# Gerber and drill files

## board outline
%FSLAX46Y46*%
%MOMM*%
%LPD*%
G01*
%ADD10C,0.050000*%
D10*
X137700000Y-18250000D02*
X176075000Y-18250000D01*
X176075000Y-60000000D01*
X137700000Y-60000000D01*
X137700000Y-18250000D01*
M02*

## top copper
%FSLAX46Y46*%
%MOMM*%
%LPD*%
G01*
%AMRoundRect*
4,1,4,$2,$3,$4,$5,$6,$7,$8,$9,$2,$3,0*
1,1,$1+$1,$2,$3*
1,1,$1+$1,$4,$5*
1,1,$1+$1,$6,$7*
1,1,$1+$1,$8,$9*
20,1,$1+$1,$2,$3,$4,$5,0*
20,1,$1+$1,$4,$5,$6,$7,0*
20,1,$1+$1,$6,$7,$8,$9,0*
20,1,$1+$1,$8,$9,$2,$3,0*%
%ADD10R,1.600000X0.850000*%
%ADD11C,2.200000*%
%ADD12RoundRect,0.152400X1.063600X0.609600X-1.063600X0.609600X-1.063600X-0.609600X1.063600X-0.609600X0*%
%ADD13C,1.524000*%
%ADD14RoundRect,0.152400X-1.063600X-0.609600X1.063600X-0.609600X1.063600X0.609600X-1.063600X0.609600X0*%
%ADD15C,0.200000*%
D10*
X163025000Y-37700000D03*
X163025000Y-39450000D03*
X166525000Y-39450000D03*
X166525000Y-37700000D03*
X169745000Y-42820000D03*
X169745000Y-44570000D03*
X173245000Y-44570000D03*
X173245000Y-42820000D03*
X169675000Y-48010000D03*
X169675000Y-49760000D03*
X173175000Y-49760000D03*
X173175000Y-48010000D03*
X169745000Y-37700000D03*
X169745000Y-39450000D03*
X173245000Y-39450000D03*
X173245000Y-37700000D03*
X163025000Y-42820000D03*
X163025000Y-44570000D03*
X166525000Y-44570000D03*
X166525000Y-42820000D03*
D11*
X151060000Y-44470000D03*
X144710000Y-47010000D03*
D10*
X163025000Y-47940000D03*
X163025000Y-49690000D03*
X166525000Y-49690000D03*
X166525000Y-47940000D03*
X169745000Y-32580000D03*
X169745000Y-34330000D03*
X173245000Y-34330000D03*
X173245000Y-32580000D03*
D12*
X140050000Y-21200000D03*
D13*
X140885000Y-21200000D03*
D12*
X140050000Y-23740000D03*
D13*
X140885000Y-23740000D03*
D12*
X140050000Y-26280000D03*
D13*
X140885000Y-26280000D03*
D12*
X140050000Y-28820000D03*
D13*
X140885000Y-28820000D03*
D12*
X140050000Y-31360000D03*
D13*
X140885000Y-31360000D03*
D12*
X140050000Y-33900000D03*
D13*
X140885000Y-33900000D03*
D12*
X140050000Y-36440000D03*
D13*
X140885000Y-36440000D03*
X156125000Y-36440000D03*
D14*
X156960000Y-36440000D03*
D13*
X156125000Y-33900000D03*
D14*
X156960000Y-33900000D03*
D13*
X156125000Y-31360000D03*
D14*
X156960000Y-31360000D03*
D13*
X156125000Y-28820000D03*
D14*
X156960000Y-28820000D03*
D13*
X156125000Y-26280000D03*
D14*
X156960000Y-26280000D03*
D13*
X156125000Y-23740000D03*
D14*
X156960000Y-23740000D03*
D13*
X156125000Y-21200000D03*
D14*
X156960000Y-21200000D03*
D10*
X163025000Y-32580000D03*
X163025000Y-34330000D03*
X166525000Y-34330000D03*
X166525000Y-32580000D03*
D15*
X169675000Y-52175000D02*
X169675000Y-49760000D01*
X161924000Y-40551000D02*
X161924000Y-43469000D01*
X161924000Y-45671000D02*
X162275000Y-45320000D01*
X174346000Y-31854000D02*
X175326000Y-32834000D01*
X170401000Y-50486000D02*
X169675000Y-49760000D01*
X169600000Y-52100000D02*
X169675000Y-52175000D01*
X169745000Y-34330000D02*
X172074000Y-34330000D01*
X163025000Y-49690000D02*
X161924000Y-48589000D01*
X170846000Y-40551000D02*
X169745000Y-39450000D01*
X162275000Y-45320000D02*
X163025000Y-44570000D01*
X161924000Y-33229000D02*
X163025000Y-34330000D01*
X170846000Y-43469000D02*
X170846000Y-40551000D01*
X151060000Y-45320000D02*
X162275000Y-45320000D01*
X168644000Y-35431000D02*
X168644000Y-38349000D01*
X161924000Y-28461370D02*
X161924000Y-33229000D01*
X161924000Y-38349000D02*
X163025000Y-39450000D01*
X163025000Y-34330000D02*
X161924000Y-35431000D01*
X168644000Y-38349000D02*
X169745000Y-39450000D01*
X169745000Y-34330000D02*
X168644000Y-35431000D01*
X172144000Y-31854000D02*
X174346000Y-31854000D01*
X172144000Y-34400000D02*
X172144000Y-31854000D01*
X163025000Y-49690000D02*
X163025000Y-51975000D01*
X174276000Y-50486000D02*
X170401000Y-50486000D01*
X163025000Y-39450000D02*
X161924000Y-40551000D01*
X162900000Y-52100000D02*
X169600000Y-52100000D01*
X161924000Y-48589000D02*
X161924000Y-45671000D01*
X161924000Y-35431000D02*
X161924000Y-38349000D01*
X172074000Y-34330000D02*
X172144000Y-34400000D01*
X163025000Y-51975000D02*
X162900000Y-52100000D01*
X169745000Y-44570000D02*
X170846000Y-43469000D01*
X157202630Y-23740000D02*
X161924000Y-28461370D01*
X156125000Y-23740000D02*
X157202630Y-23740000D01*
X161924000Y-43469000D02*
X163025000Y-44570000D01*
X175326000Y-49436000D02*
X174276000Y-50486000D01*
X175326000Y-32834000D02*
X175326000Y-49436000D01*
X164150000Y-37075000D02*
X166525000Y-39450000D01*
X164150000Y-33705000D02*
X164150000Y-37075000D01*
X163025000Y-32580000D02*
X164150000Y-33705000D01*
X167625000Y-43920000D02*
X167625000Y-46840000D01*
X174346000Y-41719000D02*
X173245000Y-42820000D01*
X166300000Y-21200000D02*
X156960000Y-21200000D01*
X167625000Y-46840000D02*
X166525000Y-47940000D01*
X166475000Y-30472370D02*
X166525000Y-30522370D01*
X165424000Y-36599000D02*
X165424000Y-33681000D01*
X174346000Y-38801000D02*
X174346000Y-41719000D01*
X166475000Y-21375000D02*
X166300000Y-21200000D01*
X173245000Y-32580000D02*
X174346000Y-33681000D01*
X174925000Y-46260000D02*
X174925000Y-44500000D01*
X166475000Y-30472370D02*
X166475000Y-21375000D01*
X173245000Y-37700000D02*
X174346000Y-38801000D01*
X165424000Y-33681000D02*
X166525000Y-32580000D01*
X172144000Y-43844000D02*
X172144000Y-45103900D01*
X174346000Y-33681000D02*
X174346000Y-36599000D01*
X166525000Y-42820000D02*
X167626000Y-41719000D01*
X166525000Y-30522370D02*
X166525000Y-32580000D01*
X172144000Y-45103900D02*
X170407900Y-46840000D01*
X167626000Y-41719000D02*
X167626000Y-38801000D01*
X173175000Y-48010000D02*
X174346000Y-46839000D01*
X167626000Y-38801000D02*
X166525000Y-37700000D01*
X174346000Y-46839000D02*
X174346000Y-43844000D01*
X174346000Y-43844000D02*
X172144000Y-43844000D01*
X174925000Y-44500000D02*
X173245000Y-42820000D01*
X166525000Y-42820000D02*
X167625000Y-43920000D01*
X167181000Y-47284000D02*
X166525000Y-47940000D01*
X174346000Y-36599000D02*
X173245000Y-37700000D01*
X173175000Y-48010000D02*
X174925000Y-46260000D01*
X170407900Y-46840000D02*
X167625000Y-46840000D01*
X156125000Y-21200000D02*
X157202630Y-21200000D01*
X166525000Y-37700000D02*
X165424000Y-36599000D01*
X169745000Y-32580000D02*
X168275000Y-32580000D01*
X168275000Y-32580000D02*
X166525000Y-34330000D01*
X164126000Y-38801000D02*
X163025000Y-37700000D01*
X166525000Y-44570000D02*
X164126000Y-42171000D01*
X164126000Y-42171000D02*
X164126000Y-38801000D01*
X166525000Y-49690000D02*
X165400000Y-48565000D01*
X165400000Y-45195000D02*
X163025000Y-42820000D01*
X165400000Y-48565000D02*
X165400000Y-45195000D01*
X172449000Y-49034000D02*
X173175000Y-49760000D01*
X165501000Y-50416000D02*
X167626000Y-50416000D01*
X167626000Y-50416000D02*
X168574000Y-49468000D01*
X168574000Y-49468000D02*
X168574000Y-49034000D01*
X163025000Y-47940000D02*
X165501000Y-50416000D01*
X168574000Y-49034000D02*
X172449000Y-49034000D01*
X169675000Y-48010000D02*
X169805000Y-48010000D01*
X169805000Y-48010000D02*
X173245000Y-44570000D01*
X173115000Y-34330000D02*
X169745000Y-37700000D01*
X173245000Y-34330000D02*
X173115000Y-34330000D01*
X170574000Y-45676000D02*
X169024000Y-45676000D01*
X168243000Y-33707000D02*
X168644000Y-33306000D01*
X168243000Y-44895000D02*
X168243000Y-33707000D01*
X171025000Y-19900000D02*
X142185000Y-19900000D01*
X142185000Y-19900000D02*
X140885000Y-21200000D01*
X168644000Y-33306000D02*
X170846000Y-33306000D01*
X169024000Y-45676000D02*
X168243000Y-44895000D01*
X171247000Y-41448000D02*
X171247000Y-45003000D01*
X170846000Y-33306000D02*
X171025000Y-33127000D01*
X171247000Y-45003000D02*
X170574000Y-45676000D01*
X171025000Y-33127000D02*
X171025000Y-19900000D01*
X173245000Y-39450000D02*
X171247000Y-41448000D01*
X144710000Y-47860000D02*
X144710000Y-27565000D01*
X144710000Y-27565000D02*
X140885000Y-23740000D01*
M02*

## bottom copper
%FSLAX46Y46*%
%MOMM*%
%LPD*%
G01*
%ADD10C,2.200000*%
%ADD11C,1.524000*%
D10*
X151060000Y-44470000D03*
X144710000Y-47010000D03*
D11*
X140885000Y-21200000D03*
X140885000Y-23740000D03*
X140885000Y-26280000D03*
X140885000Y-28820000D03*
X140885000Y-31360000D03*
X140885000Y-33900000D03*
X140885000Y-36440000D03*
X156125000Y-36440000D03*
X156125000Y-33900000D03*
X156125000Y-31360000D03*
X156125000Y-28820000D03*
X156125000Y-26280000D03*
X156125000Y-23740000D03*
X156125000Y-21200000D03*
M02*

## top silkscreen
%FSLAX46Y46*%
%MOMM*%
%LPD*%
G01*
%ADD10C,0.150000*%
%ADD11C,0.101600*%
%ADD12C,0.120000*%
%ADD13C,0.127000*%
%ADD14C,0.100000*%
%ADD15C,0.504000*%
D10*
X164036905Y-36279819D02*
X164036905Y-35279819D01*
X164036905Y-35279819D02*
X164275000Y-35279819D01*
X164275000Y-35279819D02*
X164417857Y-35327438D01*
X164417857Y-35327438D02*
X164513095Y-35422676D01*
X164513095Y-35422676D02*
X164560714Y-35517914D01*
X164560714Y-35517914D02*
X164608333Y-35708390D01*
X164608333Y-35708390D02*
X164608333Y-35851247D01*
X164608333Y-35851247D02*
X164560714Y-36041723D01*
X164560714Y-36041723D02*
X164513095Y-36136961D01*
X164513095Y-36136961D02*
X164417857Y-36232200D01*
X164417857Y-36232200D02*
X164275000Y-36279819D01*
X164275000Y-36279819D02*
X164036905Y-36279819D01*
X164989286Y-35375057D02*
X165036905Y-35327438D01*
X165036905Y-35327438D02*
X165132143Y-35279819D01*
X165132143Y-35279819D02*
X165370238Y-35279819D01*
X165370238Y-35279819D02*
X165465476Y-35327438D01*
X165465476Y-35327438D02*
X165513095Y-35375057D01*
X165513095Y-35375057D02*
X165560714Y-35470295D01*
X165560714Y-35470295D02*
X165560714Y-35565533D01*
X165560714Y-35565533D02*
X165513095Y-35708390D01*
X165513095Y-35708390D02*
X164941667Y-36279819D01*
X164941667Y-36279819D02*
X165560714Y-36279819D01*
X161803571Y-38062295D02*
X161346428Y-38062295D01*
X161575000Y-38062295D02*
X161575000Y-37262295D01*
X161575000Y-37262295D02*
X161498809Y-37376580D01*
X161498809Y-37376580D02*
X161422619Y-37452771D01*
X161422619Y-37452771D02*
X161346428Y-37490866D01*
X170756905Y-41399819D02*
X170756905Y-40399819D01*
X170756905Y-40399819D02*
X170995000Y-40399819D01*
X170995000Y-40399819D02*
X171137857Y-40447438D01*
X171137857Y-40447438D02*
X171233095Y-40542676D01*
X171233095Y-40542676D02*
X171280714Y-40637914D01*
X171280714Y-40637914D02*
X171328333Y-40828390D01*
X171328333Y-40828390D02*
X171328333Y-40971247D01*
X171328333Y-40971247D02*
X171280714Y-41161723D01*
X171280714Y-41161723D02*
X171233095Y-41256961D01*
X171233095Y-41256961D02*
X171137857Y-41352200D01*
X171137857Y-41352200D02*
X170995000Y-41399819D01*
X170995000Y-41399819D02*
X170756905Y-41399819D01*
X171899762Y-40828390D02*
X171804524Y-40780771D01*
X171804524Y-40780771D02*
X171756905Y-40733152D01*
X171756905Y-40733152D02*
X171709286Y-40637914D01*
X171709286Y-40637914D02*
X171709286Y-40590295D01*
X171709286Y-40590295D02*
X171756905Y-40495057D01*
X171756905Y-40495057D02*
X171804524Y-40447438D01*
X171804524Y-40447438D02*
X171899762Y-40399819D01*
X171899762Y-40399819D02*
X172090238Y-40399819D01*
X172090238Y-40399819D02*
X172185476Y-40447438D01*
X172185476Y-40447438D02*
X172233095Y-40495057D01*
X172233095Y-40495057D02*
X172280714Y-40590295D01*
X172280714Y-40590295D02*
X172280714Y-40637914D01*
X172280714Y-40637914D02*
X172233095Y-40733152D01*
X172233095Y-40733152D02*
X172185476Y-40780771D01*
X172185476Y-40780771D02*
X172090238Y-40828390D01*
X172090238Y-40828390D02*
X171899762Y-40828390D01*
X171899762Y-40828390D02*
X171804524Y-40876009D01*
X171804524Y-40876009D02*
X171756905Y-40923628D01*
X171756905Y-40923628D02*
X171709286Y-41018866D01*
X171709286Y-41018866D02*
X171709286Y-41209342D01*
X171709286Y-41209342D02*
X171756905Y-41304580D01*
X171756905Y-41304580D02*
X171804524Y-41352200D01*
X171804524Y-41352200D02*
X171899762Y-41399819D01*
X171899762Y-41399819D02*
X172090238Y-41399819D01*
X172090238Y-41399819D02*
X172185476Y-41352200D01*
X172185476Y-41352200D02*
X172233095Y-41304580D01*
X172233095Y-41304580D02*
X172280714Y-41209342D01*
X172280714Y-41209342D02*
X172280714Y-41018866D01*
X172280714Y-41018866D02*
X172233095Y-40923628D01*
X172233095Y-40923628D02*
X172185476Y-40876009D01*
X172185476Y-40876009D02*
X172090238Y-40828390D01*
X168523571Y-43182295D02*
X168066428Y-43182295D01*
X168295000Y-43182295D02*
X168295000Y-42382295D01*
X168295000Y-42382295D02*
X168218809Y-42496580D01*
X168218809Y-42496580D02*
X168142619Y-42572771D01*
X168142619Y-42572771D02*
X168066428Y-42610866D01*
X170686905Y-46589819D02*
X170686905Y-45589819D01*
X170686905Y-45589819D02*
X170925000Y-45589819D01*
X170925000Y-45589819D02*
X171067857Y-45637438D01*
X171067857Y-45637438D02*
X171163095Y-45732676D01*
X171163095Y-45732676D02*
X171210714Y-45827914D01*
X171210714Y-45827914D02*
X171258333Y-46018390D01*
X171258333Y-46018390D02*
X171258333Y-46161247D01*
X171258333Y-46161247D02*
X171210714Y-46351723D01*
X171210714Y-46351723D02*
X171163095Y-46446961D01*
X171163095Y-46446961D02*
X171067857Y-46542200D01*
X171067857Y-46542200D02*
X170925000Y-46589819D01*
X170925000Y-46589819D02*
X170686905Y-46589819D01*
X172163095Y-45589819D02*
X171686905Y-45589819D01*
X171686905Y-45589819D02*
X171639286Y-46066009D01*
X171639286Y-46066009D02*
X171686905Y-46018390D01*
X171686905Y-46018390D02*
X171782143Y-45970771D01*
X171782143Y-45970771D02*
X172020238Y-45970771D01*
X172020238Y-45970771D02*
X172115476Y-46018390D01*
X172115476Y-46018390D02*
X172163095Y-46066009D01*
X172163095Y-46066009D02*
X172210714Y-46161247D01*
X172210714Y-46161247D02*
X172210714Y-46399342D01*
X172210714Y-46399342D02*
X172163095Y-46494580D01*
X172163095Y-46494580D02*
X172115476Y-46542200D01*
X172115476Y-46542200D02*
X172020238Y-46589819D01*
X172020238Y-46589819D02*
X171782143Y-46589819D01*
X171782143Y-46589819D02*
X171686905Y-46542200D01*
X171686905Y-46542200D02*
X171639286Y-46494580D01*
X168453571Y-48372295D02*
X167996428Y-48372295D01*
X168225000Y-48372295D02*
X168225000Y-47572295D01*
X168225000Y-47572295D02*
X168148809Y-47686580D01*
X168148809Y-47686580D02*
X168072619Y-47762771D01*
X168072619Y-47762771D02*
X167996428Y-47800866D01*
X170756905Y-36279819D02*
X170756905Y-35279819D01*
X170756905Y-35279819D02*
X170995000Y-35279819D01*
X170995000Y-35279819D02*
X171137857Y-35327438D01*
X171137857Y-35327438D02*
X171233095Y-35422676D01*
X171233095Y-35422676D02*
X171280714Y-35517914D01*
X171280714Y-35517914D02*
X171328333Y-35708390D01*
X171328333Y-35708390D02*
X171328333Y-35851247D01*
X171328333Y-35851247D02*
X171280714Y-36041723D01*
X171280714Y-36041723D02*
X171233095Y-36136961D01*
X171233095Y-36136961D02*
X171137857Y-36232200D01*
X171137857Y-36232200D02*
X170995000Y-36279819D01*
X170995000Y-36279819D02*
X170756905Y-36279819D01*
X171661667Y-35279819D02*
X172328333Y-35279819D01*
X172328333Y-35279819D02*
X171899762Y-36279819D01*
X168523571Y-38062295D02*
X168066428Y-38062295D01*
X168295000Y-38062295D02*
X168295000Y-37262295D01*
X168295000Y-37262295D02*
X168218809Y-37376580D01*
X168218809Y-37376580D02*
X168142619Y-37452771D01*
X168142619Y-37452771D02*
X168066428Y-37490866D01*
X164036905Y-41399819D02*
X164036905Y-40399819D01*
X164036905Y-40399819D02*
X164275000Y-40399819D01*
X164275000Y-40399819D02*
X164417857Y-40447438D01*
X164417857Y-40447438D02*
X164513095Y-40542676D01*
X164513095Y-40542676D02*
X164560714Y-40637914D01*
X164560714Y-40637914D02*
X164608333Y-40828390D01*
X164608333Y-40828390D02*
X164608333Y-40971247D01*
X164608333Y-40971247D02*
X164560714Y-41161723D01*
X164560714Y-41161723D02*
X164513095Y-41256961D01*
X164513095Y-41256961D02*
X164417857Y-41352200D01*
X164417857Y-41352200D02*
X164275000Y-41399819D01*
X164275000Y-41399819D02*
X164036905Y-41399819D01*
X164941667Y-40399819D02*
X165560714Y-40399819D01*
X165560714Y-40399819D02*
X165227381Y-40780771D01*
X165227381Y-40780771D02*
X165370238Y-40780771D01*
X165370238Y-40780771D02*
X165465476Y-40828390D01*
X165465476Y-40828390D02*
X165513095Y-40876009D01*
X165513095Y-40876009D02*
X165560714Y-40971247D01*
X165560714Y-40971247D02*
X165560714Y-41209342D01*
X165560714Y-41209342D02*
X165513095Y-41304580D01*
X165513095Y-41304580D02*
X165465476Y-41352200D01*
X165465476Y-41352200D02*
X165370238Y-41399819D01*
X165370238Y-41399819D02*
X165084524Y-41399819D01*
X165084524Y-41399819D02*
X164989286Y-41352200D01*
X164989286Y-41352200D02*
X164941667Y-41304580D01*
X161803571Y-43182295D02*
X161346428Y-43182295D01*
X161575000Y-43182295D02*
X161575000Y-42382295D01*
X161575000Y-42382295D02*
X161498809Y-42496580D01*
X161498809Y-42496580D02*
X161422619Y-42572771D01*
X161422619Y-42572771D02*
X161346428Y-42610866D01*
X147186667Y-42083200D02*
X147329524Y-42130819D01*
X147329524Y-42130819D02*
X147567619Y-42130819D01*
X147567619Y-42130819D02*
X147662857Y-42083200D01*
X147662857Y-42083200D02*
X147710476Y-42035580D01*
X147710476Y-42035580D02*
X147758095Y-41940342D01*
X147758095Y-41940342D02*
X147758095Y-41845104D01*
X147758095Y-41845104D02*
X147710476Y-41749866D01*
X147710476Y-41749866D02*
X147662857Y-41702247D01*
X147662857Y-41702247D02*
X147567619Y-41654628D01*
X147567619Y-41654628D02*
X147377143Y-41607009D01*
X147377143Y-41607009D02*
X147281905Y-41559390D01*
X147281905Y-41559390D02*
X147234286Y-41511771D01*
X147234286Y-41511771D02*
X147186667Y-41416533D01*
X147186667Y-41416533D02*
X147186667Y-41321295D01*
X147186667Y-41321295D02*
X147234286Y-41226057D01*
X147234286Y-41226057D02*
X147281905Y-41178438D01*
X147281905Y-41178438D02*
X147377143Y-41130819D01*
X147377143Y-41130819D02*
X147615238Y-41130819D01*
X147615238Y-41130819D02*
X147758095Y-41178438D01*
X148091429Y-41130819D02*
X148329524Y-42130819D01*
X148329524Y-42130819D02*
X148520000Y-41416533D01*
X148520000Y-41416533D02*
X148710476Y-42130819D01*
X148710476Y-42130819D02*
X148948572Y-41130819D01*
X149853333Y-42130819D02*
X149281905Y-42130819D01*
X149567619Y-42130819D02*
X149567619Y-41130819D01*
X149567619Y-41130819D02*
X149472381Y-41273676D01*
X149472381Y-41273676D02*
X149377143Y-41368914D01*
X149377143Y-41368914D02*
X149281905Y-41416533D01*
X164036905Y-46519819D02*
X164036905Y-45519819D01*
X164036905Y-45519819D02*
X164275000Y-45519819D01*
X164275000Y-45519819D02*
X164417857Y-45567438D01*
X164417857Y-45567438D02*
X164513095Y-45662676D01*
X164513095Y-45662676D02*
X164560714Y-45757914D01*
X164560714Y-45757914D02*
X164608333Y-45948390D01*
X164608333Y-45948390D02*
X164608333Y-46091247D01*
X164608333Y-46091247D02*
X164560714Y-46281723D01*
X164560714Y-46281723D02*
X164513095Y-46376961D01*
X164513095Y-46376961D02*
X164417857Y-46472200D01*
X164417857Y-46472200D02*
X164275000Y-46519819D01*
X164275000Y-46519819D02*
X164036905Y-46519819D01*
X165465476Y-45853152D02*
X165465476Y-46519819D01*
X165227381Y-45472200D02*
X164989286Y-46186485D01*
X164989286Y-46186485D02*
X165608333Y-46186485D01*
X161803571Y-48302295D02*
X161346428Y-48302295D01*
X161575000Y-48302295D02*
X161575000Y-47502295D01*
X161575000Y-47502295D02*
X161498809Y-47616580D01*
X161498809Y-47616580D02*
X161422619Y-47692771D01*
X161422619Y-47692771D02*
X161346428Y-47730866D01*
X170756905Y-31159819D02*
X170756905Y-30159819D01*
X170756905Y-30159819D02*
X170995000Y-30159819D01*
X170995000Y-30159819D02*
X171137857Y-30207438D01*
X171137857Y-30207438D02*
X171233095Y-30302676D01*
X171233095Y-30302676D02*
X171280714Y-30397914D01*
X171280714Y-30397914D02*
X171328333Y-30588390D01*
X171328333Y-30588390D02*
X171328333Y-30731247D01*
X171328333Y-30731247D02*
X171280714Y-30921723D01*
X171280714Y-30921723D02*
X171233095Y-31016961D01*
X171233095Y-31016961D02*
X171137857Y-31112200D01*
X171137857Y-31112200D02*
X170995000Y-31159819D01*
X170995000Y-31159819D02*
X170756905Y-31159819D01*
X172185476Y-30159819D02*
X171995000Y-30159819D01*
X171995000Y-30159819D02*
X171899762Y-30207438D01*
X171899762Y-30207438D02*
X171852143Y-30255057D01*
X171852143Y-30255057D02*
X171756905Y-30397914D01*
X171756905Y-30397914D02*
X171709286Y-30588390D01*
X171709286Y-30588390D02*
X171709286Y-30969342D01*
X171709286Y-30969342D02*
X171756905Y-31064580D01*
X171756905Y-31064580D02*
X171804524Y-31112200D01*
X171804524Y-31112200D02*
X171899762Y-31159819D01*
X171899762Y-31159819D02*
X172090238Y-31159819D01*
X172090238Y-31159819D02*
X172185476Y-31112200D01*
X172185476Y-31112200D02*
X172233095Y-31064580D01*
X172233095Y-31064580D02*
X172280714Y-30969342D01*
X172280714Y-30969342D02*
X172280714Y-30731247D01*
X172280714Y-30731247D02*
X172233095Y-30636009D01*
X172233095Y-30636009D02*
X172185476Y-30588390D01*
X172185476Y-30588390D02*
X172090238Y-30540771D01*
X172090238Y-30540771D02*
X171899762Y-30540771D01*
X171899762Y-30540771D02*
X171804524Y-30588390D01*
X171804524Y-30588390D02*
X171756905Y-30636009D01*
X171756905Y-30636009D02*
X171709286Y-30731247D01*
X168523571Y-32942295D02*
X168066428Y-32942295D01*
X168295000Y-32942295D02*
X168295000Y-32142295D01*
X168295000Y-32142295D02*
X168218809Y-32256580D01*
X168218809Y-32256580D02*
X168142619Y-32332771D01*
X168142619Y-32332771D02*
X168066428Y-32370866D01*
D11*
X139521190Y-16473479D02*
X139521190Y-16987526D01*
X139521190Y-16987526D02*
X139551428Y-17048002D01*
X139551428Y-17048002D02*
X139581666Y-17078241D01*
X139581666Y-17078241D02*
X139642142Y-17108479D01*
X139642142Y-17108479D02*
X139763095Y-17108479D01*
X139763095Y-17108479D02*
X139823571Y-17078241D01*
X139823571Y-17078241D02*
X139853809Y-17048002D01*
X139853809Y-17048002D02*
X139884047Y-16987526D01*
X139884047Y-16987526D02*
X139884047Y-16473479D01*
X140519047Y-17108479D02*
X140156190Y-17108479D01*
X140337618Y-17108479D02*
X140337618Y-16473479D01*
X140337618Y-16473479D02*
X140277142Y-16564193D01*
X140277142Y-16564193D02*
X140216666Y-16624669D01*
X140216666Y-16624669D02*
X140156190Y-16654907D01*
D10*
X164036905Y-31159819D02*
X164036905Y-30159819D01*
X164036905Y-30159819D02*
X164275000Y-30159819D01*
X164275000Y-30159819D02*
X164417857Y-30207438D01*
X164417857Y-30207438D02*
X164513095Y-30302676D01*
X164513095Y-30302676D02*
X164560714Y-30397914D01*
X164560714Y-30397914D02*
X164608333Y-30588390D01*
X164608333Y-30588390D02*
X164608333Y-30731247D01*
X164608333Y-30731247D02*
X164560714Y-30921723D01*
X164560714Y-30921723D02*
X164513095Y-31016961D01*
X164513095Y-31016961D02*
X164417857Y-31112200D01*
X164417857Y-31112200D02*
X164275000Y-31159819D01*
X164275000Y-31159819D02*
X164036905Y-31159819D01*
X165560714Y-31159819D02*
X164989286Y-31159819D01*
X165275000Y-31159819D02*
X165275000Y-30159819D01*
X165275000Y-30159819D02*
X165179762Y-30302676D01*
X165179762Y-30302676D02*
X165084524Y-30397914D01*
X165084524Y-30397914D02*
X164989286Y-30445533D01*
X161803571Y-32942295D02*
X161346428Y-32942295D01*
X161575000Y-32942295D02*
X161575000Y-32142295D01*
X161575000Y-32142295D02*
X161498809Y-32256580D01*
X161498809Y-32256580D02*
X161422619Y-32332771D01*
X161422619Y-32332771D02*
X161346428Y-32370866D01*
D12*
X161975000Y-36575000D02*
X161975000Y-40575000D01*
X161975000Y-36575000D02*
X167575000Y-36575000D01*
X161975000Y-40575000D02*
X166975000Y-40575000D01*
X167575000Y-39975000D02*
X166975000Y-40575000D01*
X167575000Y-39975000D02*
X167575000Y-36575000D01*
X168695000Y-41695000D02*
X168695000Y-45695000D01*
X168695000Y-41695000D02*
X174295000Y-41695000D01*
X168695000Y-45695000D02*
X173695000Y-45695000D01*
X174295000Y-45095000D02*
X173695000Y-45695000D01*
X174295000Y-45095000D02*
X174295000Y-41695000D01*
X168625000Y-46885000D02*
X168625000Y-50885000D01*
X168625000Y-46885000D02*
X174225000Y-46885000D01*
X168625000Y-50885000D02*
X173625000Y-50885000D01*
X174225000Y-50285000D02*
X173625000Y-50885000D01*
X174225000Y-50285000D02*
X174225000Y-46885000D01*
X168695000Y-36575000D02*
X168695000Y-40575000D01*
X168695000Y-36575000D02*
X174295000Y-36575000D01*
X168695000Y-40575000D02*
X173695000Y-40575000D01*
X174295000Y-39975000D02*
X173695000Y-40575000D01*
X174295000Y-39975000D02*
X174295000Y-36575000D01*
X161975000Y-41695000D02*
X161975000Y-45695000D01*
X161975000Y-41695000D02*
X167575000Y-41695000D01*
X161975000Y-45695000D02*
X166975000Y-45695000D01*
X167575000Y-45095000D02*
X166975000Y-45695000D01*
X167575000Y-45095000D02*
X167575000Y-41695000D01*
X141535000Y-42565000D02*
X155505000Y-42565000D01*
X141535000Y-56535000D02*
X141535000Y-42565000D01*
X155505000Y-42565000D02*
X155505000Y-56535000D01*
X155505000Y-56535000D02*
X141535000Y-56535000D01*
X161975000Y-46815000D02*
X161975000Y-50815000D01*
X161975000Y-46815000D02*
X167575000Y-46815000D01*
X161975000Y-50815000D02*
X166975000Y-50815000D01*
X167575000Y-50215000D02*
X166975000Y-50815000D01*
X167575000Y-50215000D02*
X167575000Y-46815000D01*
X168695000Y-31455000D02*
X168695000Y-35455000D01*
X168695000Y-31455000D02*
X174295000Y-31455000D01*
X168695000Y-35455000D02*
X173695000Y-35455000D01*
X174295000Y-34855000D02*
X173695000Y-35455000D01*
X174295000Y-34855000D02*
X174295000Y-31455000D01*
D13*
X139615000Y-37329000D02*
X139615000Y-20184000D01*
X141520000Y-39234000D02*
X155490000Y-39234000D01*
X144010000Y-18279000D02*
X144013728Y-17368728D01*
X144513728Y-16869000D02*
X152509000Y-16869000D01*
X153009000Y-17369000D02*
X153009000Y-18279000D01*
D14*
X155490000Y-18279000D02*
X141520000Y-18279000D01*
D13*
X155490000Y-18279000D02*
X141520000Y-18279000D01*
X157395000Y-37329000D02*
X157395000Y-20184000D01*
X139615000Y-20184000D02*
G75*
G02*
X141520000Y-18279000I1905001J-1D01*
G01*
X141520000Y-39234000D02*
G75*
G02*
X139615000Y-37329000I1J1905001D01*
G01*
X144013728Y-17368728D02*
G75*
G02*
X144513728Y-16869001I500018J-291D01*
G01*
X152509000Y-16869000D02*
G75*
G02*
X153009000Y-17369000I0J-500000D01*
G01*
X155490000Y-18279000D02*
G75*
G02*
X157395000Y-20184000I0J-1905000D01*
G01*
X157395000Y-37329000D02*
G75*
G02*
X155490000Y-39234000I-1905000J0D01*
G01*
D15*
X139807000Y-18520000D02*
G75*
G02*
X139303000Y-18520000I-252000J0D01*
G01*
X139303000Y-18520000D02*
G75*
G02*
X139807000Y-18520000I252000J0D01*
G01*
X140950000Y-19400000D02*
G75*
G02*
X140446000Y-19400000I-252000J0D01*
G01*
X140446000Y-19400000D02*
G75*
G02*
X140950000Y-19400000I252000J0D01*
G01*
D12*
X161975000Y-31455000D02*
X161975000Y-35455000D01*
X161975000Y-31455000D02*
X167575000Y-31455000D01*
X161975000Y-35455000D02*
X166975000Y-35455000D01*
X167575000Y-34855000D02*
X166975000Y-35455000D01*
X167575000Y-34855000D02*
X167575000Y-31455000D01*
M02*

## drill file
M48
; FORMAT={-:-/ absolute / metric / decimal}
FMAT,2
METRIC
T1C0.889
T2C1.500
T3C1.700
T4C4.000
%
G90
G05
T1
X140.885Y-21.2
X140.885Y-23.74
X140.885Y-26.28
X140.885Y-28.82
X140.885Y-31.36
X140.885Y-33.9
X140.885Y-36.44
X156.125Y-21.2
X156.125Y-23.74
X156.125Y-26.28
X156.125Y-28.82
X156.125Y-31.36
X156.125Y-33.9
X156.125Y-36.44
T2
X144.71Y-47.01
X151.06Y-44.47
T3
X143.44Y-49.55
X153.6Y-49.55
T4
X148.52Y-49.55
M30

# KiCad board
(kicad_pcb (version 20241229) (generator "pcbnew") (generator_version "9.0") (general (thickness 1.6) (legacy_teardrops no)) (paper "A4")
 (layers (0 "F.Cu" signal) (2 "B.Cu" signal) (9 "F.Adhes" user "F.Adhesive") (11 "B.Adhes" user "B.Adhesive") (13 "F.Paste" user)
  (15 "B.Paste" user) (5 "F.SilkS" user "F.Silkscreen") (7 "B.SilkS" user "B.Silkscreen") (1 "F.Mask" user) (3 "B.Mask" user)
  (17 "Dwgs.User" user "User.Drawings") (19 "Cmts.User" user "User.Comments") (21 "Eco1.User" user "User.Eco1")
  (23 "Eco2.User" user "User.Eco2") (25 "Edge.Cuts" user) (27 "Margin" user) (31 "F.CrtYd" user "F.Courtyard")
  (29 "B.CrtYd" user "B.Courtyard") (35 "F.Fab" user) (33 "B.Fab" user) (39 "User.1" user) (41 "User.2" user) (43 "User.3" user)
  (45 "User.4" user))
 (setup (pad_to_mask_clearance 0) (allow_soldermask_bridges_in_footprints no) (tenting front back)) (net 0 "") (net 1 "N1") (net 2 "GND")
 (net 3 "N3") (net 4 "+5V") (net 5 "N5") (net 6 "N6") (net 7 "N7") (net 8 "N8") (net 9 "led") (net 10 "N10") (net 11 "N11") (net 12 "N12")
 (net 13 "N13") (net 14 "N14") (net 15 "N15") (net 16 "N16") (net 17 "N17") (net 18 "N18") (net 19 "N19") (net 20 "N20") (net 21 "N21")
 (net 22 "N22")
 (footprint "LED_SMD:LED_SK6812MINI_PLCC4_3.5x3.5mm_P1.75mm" (layer "F.Cu") (at 164.775 38.575)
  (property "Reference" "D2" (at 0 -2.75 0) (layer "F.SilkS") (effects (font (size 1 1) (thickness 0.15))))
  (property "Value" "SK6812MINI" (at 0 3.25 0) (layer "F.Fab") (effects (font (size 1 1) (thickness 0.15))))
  (fp_line (start -2.8 -2) (end -2.8 2) (stroke (width 0.12) (type default)) (layer "F.SilkS"))
  (fp_line (start -2.8 -2) (end 2.8 -2) (stroke (width 0.12) (type solid)) (layer "F.SilkS"))
  (fp_line (start -2.8 2) (end 2.2 2) (stroke (width 0.12) (type solid)) (layer "F.SilkS"))
  (fp_line (start 2.8 1.4) (end 2.2 2) (stroke (width 0.12) (type default)) (layer "F.SilkS"))
  (fp_line (start 2.8 1.4) (end 2.8 -2) (stroke (width 0.12) (type solid)) (layer "F.SilkS"))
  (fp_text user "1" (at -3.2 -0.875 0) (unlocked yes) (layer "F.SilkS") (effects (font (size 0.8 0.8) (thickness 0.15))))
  (pad "1" smd rect (at -1.75 -0.875) (size 1.6 0.85) (layers "F.Cu" "F.Mask" "F.Paste") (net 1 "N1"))
  (pad "2" smd rect (at -1.75 0.875) (size 1.6 0.85) (layers "F.Cu" "F.Mask" "F.Paste") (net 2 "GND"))
  (pad "3" smd rect (at 1.75 0.875) (size 1.6 0.85) (layers "F.Cu" "F.Mask" "F.Paste") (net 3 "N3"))
  (pad "4" smd rect (at 1.75 -0.875) (size 1.6 0.85) (layers "F.Cu" "F.Mask" "F.Paste") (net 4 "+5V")))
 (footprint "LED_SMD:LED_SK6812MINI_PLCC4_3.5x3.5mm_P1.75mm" (layer "F.Cu") (at 171.495 43.695)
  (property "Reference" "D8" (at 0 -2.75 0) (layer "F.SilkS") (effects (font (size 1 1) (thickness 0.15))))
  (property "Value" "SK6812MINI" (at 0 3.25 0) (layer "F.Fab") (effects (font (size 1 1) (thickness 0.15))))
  (fp_line (start -2.8 -2) (end -2.8 2) (stroke (width 0.12) (type default)) (layer "F.SilkS"))
  (fp_line (start -2.8 -2) (end 2.8 -2) (stroke (width 0.12) (type solid)) (layer "F.SilkS"))
  (fp_line (start -2.8 2) (end 2.2 2) (stroke (width 0.12) (type solid)) (layer "F.SilkS"))
  (fp_line (start 2.8 1.4) (end 2.2 2) (stroke (width 0.12) (type default)) (layer "F.SilkS"))
  (fp_line (start 2.8 1.4) (end 2.8 -2) (stroke (width 0.12) (type solid)) (layer "F.SilkS"))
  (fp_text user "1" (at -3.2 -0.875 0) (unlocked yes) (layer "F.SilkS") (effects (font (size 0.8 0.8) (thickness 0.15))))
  (pad "1" smd rect (at -1.75 -0.875) (size 1.6 0.85) (layers "F.Cu" "F.Mask" "F.Paste") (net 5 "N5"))
  (pad "2" smd rect (at -1.75 0.875) (size 1.6 0.85) (layers "F.Cu" "F.Mask" "F.Paste") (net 2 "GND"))
  (pad "3" smd rect (at 1.75 0.875) (size 1.6 0.85) (layers "F.Cu" "F.Mask" "F.Paste") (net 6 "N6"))
  (pad "4" smd rect (at 1.75 -0.875) (size 1.6 0.85) (layers "F.Cu" "F.Mask" "F.Paste") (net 4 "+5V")))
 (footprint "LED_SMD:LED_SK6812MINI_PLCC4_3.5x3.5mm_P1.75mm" (layer "F.Cu") (at 171.425 48.885)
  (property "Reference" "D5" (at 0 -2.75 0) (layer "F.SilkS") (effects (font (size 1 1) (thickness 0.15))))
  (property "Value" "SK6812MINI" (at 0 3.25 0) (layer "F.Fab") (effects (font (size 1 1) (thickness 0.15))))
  (fp_line (start -2.8 -2) (end -2.8 2) (stroke (width 0.12) (type default)) (layer "F.SilkS"))
  (fp_line (start -2.8 -2) (end 2.8 -2) (stroke (width 0.12) (type solid)) (layer "F.SilkS"))
  (fp_line (start -2.8 2) (end 2.2 2) (stroke (width 0.12) (type solid)) (layer "F.SilkS"))
  (fp_line (start 2.8 1.4) (end 2.2 2) (stroke (width 0.12) (type default)) (layer "F.SilkS"))
  (fp_line (start 2.8 1.4) (end 2.8 -2) (stroke (width 0.12) (type solid)) (layer "F.SilkS"))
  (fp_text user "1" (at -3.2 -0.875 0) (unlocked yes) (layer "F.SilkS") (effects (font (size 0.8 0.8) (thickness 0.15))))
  (pad "1" smd rect (at -1.75 -0.875) (size 1.6 0.85) (layers "F.Cu" "F.Mask" "F.Paste") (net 6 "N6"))
  (pad "2" smd rect (at -1.75 0.875) (size 1.6 0.85) (layers "F.Cu" "F.Mask" "F.Paste") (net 2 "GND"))
  (pad "3" smd rect (at 1.75 0.875) (size 1.6 0.85) (layers "F.Cu" "F.Mask" "F.Paste") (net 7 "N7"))
  (pad "4" smd rect (at 1.75 -0.875) (size 1.6 0.85) (layers "F.Cu" "F.Mask" "F.Paste") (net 4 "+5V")))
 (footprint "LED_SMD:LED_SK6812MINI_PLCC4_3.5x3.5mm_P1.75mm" (layer "F.Cu") (at 171.495 38.575)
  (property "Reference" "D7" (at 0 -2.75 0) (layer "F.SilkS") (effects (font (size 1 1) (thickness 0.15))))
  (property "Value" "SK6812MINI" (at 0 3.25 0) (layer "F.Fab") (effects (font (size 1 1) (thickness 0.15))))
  (fp_line (start -2.8 -2) (end -2.8 2) (stroke (width 0.12) (type default)) (layer "F.SilkS"))
  (fp_line (start -2.8 -2) (end 2.8 -2) (stroke (width 0.12) (type solid)) (layer "F.SilkS"))
  (fp_line (start -2.8 2) (end 2.2 2) (stroke (width 0.12) (type solid)) (layer "F.SilkS"))
  (fp_line (start 2.8 1.4) (end 2.2 2) (stroke (width 0.12) (type default)) (layer "F.SilkS"))
  (fp_line (start 2.8 1.4) (end 2.8 -2) (stroke (width 0.12) (type solid)) (layer "F.SilkS"))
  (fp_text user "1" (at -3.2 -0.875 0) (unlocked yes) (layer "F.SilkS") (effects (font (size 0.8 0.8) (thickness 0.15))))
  (pad "1" smd rect (at -1.75 -0.875) (size 1.6 0.85) (layers "F.Cu" "F.Mask" "F.Paste") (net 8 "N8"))
  (pad "2" smd rect (at -1.75 0.875) (size 1.6 0.85) (layers "F.Cu" "F.Mask" "F.Paste") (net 2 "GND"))
  (pad "3" smd rect (at 1.75 0.875) (size 1.6 0.85) (layers "F.Cu" "F.Mask" "F.Paste") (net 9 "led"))
  (pad "4" smd rect (at 1.75 -0.875) (size 1.6 0.85) (layers "F.Cu" "F.Mask" "F.Paste") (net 4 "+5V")))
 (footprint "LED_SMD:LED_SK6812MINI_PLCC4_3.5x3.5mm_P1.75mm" (layer "F.Cu") (at 164.775 43.695)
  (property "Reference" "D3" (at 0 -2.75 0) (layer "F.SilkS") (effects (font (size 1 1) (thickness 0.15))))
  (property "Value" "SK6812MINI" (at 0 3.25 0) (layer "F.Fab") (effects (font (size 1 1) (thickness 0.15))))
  (fp_line (start -2.8 -2) (end -2.8 2) (stroke (width 0.12) (type default)) (layer "F.SilkS"))
  (fp_line (start -2.8 -2) (end 2.8 -2) (stroke (width 0.12) (type solid)) (layer "F.SilkS"))
  (fp_line (start -2.8 2) (end 2.2 2) (stroke (width 0.12) (type solid)) (layer "F.SilkS"))
  (fp_line (start 2.8 1.4) (end 2.2 2) (stroke (width 0.12) (type default)) (layer "F.SilkS"))
  (fp_line (start 2.8 1.4) (end 2.8 -2) (stroke (width 0.12) (type solid)) (layer "F.SilkS"))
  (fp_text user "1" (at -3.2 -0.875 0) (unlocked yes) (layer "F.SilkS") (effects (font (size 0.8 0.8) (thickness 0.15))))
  (pad "1" smd rect (at -1.75 -0.875) (size 1.6 0.85) (layers "F.Cu" "F.Mask" "F.Paste") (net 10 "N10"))
  (pad "2" smd rect (at -1.75 0.875) (size 1.6 0.85) (layers "F.Cu" "F.Mask" "F.Paste") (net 2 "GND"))
  (pad "3" smd rect (at 1.75 0.875) (size 1.6 0.85) (layers "F.Cu" "F.Mask" "F.Paste") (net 1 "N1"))
  (pad "4" smd rect (at 1.75 -0.875) (size 1.6 0.85) (layers "F.Cu" "F.Mask" "F.Paste") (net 4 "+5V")))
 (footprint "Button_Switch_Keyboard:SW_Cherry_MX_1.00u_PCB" (layer "F.Cu") (at 151.06 44.47)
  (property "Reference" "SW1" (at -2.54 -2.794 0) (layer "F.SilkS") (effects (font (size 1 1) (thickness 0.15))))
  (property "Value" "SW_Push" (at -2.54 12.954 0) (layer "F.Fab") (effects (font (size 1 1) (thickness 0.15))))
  (fp_line (start -9.525 -1.905) (end 4.445 -1.905) (stroke (width 0.12) (type solid)) (layer "F.SilkS"))
  (fp_line (start -9.525 12.065) (end -9.525 -1.905) (stroke (width 0.12) (type solid)) (layer "F.SilkS"))
  (fp_line (start 4.445 -1.905) (end 4.445 12.065) (stroke (width 0.12) (type solid)) (layer "F.SilkS"))
  (fp_line (start 4.445 12.065) (end -9.525 12.065) (stroke (width 0.12) (type solid)) (layer "F.SilkS"))
  (pad "" np_thru_hole circle (at -7.62 5.08) (size 1.7 1.7) (drill 1.7) (layers "*.Cu" "*.Mask"))
  (pad "" np_thru_hole circle (at -2.54 5.08) (size 4 4) (drill 4) (layers "*.Cu" "*.Mask"))
  (pad "" np_thru_hole circle (at 2.54 5.08) (size 1.7 1.7) (drill 1.7) (layers "*.Cu" "*.Mask"))
  (pad "1" thru_hole circle (at 0 0) (size 2.2 2.2) (drill 1.5) (layers "*.Cu" "*.Mask") (remove_unused_layers no) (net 2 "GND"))
  (pad "2" thru_hole circle (at -6.35 2.54) (size 2.2 2.2) (drill 1.5) (layers "*.Cu" "*.Mask") (remove_unused_layers no) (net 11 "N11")))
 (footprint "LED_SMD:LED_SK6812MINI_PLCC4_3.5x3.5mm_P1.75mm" (layer "F.Cu") (at 164.775 48.815)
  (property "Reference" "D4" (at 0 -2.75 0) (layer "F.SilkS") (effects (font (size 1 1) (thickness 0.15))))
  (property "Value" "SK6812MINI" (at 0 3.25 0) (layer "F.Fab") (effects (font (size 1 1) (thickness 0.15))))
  (fp_line (start -2.8 -2) (end -2.8 2) (stroke (width 0.12) (type default)) (layer "F.SilkS"))
  (fp_line (start -2.8 -2) (end 2.8 -2) (stroke (width 0.12) (type solid)) (layer "F.SilkS"))
  (fp_line (start -2.8 2) (end 2.2 2) (stroke (width 0.12) (type solid)) (layer "F.SilkS"))
  (fp_line (start 2.8 1.4) (end 2.2 2) (stroke (width 0.12) (type default)) (layer "F.SilkS"))
  (fp_line (start 2.8 1.4) (end 2.8 -2) (stroke (width 0.12) (type solid)) (layer "F.SilkS"))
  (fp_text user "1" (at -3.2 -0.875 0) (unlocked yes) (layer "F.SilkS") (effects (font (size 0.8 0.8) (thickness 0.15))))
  (pad "1" smd rect (at -1.75 -0.875) (size 1.6 0.85) (layers "F.Cu" "F.Mask" "F.Paste") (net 7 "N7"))
  (pad "2" smd rect (at -1.75 0.875) (size 1.6 0.85) (layers "F.Cu" "F.Mask" "F.Paste") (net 2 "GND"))
  (pad "3" smd rect (at 1.75 0.875) (size 1.6 0.85) (layers "F.Cu" "F.Mask" "F.Paste") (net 10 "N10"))
  (pad "4" smd rect (at 1.75 -0.875) (size 1.6 0.85) (layers "F.Cu" "F.Mask" "F.Paste") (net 4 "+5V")))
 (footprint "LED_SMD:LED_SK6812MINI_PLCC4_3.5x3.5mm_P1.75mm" (layer "F.Cu") (at 171.495 33.455)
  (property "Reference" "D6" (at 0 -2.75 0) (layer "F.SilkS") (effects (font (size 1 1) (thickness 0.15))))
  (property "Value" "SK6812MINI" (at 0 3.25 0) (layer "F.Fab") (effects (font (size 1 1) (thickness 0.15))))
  (fp_line (start -2.8 -2) (end -2.8 2) (stroke (width 0.12) (type default)) (layer "F.SilkS"))
  (fp_line (start -2.8 -2) (end 2.8 -2) (stroke (width 0.12) (type solid)) (layer "F.SilkS"))
  (fp_line (start -2.8 2) (end 2.2 2) (stroke (width 0.12) (type solid)) (layer "F.SilkS"))
  (fp_line (start 2.8 1.4) (end 2.2 2) (stroke (width 0.12) (type default)) (layer "F.SilkS"))
  (fp_line (start 2.8 1.4) (end 2.8 -2) (stroke (width 0.12) (type solid)) (layer "F.SilkS"))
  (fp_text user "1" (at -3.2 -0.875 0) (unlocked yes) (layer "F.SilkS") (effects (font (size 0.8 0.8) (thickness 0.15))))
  (pad "1" smd rect (at -1.75 -0.875) (size 1.6 0.85) (layers "F.Cu" "F.Mask" "F.Paste") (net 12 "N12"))
  (pad "2" smd rect (at -1.75 0.875) (size 1.6 0.85) (layers "F.Cu" "F.Mask" "F.Paste") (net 2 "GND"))
  (pad "3" smd rect (at 1.75 0.875) (size 1.6 0.85) (layers "F.Cu" "F.Mask" "F.Paste") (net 8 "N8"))
  (pad "4" smd rect (at 1.75 -0.875) (size 1.6 0.85) (layers "F.Cu" "F.Mask" "F.Paste") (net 4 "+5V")))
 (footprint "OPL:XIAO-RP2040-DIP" (layer "F.Cu") (at 148.505 28.82)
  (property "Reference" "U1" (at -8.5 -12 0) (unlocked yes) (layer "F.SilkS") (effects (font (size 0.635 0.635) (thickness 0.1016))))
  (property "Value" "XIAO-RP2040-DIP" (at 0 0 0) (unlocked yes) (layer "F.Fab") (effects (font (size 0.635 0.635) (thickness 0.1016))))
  (fp_line (start -8.89 8.509) (end -8.89 -8.636) (stroke (width 0.127) (type solid)) (layer "F.SilkS"))
  (fp_line (start -6.985 10.414) (end 6.985 10.414) (stroke (width 0.127) (type solid)) (layer "F.SilkS"))
  (fp_line (start -4.495 -10.541) (end -4.491272 -11.451272) (stroke (width 0.127) (type solid)) (layer "F.SilkS"))
  (fp_line (start -3.991272 -11.951) (end 4.004 -11.951) (stroke (width 0.127) (type solid)) (layer "F.SilkS"))
  (fp_line (start 4.504 -11.451) (end 4.504 -10.541) (stroke (width 0.127) (type solid)) (layer "F.SilkS"))
  (fp_line (start 6.985 -10.541) (end -6.985 -10.541) (stroke (width 0.1) (type solid)) (layer "F.SilkS"))
  (fp_line (start 6.985 -10.541) (end -6.985 -10.541) (stroke (width 0.127) (type solid)) (layer "F.SilkS"))
  (fp_line (start 8.89 8.509) (end 8.89 -8.636) (stroke (width 0.127) (type solid)) (layer "F.SilkS"))
  (fp_arc (start -8.89 -8.636) (mid -8.332038 -9.983038) (end -6.985 -10.541) (stroke (width 0.127) (type solid)) (layer "F.SilkS"))
  (fp_arc (start -6.985 10.414) (mid -8.332038 9.856038) (end -8.89 8.509) (stroke (width 0.127) (type solid)) (layer "F.SilkS"))
  (fp_arc (start -4.491272 -11.451272) (mid -4.344728 -11.80464) (end -3.991272 -11.951) (stroke (width 0.127) (type default))
   (layer "F.SilkS"))
  (fp_arc (start 4.004 -11.951) (mid 4.357553 -11.804553) (end 4.504 -11.451) (stroke (width 0.127) (type default)) (layer "F.SilkS"))
  (fp_arc (start 6.985 -10.541) (mid 8.332038 -9.983038) (end 8.89 -8.636) (stroke (width 0.127) (type solid)) (layer "F.SilkS"))
  (fp_arc (start 8.89 8.509) (mid 8.332038 9.856038) (end 6.985 10.414) (stroke (width 0.127) (type solid)) (layer "F.SilkS"))
  (fp_circle (center -8.95 -10.3) (end -8.95 -10.554) (stroke (width 0.5) (type solid)) (fill yes) (layer "F.SilkS"))
  (fp_circle (center -7.807 -9.42) (end -7.807 -9.674) (stroke (width 0.5) (type solid)) (fill yes) (layer "F.SilkS"))
  (pad "1" smd roundrect (at -8.455 -7.62 180) (size 2.432 1.524) (layers "F.Cu" "F.Mask") (roundrect_rratio 0.1) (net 9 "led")
   (thermal_bridge_angle 45))
  (pad "1" thru_hole circle (at -7.62 -7.62 180) (size 1.524 1.524) (drill 0.889) (layers "*.Cu" "*.Mask") (remove_unused_layers no)
   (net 9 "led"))
  (pad "2" smd roundrect (at -8.455 -5.08 180) (size 2.432 1.524) (layers "F.Cu" "F.Mask") (roundrect_rratio 0.1) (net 11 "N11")
   (thermal_bridge_angle 45))
  (pad "2" thru_hole circle (at -7.62 -5.08 180) (size 1.524 1.524) (drill 0.889) (layers "*.Cu" "*.Mask") (remove_unused_layers no)
   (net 11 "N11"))
  (pad "3" smd roundrect (at -8.455 -2.54 180) (size 2.432 1.524) (layers "F.Cu" "F.Mask") (roundrect_rratio 0.1) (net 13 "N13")
   (thermal_bridge_angle 45))
  (pad "3" thru_hole circle (at -7.62 -2.54 180) (size 1.524 1.524) (drill 0.889) (layers "*.Cu" "*.Mask") (remove_unused_layers no)
   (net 13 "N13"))
  (pad "4" smd roundrect (at -8.455 0 180) (size 2.432 1.524) (layers "F.Cu" "F.Mask") (roundrect_rratio 0.1) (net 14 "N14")
   (thermal_bridge_angle 45))
  (pad "4" thru_hole circle (at -7.62 0 180) (size 1.524 1.524) (drill 0.889) (layers "*.Cu" "*.Mask") (remove_unused_layers no)
   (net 14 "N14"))
  (pad "5" smd roundrect (at -8.455 2.54 180) (size 2.432 1.524) (layers "F.Cu" "F.Mask") (roundrect_rratio 0.1) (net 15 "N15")
   (thermal_bridge_angle 45))
  (pad "5" thru_hole circle (at -7.62 2.54 180) (size 1.524 1.524) (drill 0.889) (layers "*.Cu" "*.Mask") (remove_unused_layers no)
   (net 15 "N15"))
  (pad "6" smd roundrect (at -8.455 5.08 180) (size 2.432 1.524) (layers "F.Cu" "F.Mask") (roundrect_rratio 0.1) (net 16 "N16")
   (thermal_bridge_angle 45))
  (pad "6" thru_hole circle (at -7.62 5.08 180) (size 1.524 1.524) (drill 0.889) (layers "*.Cu" "*.Mask") (remove_unused_layers no)
   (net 16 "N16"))
  (pad "7" smd roundrect (at -8.455 7.62 180) (size 2.432 1.524) (layers "F.Cu" "F.Mask") (roundrect_rratio 0.1) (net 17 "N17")
   (thermal_bridge_angle 45))
  (pad "7" thru_hole circle (at -7.62 7.62 180) (size 1.524 1.524) (drill 0.889) (layers "*.Cu" "*.Mask") (remove_unused_layers no)
   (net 17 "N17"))
  (pad "8" thru_hole circle (at 7.62 7.62) (size 1.524 1.524) (drill 0.889) (layers "*.Cu" "*.Mask") (remove_unused_layers no)
   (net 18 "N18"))
  (pad "8" smd roundrect (at 8.455 7.62) (size 2.432 1.524) (layers "F.Cu" "F.Mask") (roundrect_rratio 0.1) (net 18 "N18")
   (thermal_bridge_angle 45))
  (pad "9" thru_hole circle (at 7.62 5.08) (size 1.524 1.524) (drill 0.889) (layers "*.Cu" "*.Mask") (remove_unused_layers no)
   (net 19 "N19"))
  (pad "9" smd roundrect (at 8.455 5.08) (size 2.432 1.524) (layers "F.Cu" "F.Mask") (roundrect_rratio 0.1) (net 19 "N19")
   (thermal_bridge_angle 45))
  (pad "10" thru_hole circle (at 7.62 2.54) (size 1.524 1.524) (drill 0.889) (layers "*.Cu" "*.Mask") (remove_unused_layers no)
   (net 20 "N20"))
  (pad "10" smd roundrect (at 8.455 2.54) (size 2.432 1.524) (layers "F.Cu" "F.Mask") (roundrect_rratio 0.1) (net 20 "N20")
   (thermal_bridge_angle 45))
  (pad "11" thru_hole circle (at 7.62 0) (size 1.524 1.524) (drill 0.889) (layers "*.Cu" "*.Mask") (remove_unused_layers no) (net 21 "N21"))
  (pad "11" smd roundrect (at 8.455 0) (size 2.432 1.524) (layers "F.Cu" "F.Mask") (roundrect_rratio 0.1) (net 21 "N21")
   (thermal_bridge_angle 45))
  (pad "12" thru_hole circle (at 7.62 -2.54) (size 1.524 1.524) (drill 0.889) (layers "*.Cu" "*.Mask") (remove_unused_layers no)
   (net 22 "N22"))
  (pad "12" smd roundrect (at 8.455 -2.54) (size 2.432 1.524) (layers "F.Cu" "F.Mask") (roundrect_rratio 0.1) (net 22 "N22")
   (thermal_bridge_angle 45))
  (pad "13" thru_hole circle (at 7.62 -5.08) (size 1.524 1.524) (drill 0.889) (layers "*.Cu" "*.Mask") (remove_unused_layers no)
   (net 2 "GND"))
  (pad "13" smd roundrect (at 8.455 -5.08) (size 2.432 1.524) (layers "F.Cu" "F.Mask") (roundrect_rratio 0.1) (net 2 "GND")
   (thermal_bridge_angle 45))
  (pad "14" thru_hole circle (at 7.62 -7.62) (size 1.524 1.524) (drill 0.889) (layers "*.Cu" "*.Mask") (remove_unused_layers no)
   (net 4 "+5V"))
  (pad "14" smd roundrect (at 8.455 -7.62) (size 2.432 1.524) (layers "F.Cu" "F.Mask") (roundrect_rratio 0.1) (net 4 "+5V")
   (thermal_bridge_angle 45)))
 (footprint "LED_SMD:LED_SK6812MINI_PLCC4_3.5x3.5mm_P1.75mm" (layer "F.Cu") (at 164.775 33.455)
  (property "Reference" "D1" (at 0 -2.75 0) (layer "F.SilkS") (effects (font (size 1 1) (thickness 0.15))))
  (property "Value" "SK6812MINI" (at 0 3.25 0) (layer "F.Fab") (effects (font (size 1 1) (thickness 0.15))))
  (fp_line (start -2.8 -2) (end -2.8 2) (stroke (width 0.12) (type default)) (layer "F.SilkS"))
  (fp_line (start -2.8 -2) (end 2.8 -2) (stroke (width 0.12) (type solid)) (layer "F.SilkS"))
  (fp_line (start -2.8 2) (end 2.2 2) (stroke (width 0.12) (type solid)) (layer "F.SilkS"))
  (fp_line (start 2.8 1.4) (end 2.2 2) (stroke (width 0.12) (type default)) (layer "F.SilkS"))
  (fp_line (start 2.8 1.4) (end 2.8 -2) (stroke (width 0.12) (type solid)) (layer "F.SilkS"))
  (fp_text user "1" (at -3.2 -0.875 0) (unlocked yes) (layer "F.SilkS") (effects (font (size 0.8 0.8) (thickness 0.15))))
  (pad "1" smd rect (at -1.75 -0.875) (size 1.6 0.85) (layers "F.Cu" "F.Mask" "F.Paste") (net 3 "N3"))
  (pad "2" smd rect (at -1.75 0.875) (size 1.6 0.85) (layers "F.Cu" "F.Mask" "F.Paste") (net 2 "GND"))
  (pad "3" smd rect (at 1.75 0.875) (size 1.6 0.85) (layers "F.Cu" "F.Mask" "F.Paste") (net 12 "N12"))
  (pad "4" smd rect (at 1.75 -0.875) (size 1.6 0.85) (layers "F.Cu" "F.Mask" "F.Paste") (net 4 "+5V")))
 (gr_rect (start 137.7 18.25) (end 176.075 60) (stroke (width 0.05) (type default)) (fill no) (layer "Edge.Cuts"))
 (segment (start 169.675 52.175) (end 169.675 49.76) (width 0.2) (layer "F.Cu") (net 2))
 (segment (start 161.924 40.551) (end 161.924 43.469) (width 0.2) (layer "F.Cu") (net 2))
 (segment (start 161.924 45.671) (end 162.275 45.32) (width 0.2) (layer "F.Cu") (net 2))
 (segment (start 174.346 31.854) (end 175.326 32.834) (width 0.2) (layer "F.Cu") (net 2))
 (segment (start 170.401 50.486) (end 169.675 49.76) (width 0.2) (layer "F.Cu") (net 2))
 (segment (start 169.6 52.1) (end 169.675 52.175) (width 0.2) (layer "F.Cu") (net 2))
 (segment (start 169.745 34.33) (end 172.074 34.33) (width 0.2) (layer "F.Cu") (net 2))
 (segment (start 163.025 49.69) (end 161.924 48.589) (width 0.2) (layer "F.Cu") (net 2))
 (segment (start 170.846 40.551) (end 169.745 39.45) (width 0.2) (layer "F.Cu") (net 2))
 (segment (start 162.275 45.32) (end 163.025 44.57) (width 0.2) (layer "F.Cu") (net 2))
 (segment (start 161.924 33.229) (end 163.025 34.33) (width 0.2) (layer "F.Cu") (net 2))
 (segment (start 170.846 43.469) (end 170.846 40.551) (width 0.2) (layer "F.Cu") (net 2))
 (segment (start 151.06 45.32) (end 162.275 45.32) (width 0.2) (layer "F.Cu") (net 2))
 (segment (start 168.644 35.431) (end 168.644 38.349) (width 0.2) (layer "F.Cu") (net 2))
 (segment (start 161.924 28.46137) (end 161.924 33.229) (width 0.2) (layer "F.Cu") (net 2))
 (segment (start 161.924 38.349) (end 163.025 39.45) (width 0.2) (layer "F.Cu") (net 2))
 (segment (start 163.025 34.33) (end 161.924 35.431) (width 0.2) (layer "F.Cu") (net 2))
 (segment (start 168.644 38.349) (end 169.745 39.45) (width 0.2) (layer "F.Cu") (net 2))
 (segment (start 169.745 34.33) (end 168.644 35.431) (width 0.2) (layer "F.Cu") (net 2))
 (segment (start 172.144 31.854) (end 174.346 31.854) (width 0.2) (layer "F.Cu") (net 2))
 (segment (start 172.144 34.4) (end 172.144 31.854) (width 0.2) (layer "F.Cu") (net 2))
 (segment (start 163.025 49.69) (end 163.025 51.975) (width 0.2) (layer "F.Cu") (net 2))
 (segment (start 174.276 50.486) (end 170.401 50.486) (width 0.2) (layer "F.Cu") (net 2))
 (segment (start 163.025 39.45) (end 161.924 40.551) (width 0.2) (layer "F.Cu") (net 2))
 (segment (start 162.9 52.1) (end 169.6 52.1) (width 0.2) (layer "F.Cu") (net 2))
 (segment (start 161.924 48.589) (end 161.924 45.671) (width 0.2) (layer "F.Cu") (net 2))
 (segment (start 161.924 35.431) (end 161.924 38.349) (width 0.2) (layer "F.Cu") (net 2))
 (segment (start 172.074 34.33) (end 172.144 34.4) (width 0.2) (layer "F.Cu") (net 2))
 (segment (start 163.025 51.975) (end 162.9 52.1) (width 0.2) (layer "F.Cu") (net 2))
 (segment (start 169.745 44.57) (end 170.846 43.469) (width 0.2) (layer "F.Cu") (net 2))
 (segment (start 157.20263 23.74) (end 161.924 28.46137) (width 0.2) (layer "F.Cu") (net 2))
 (segment (start 156.125 23.74) (end 157.20263 23.74) (width 0.2) (layer "F.Cu") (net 2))
 (segment (start 161.924 43.469) (end 163.025 44.57) (width 0.2) (layer "F.Cu") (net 2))
 (segment (start 175.326 49.436) (end 174.276 50.486) (width 0.2) (layer "F.Cu") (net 2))
 (segment (start 175.326 32.834) (end 175.326 49.436) (width 0.2) (layer "F.Cu") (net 2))
 (segment (start 164.15 37.075) (end 166.525 39.45) (width 0.2) (layer "F.Cu") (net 3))
 (segment (start 164.15 33.705) (end 164.15 37.075) (width 0.2) (layer "F.Cu") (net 3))
 (segment (start 163.025 32.58) (end 164.15 33.705) (width 0.2) (layer "F.Cu") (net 3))
 (segment (start 167.625 43.92) (end 167.625 46.84) (width 0.2) (layer "F.Cu") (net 4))
 (segment (start 174.346 41.719) (end 173.245 42.82) (width 0.2) (layer "F.Cu") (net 4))
 (segment (start 166.3 21.2) (end 156.96 21.2) (width 0.2) (layer "F.Cu") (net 4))
 (segment (start 167.625 46.84) (end 166.525 47.94) (width 0.2) (layer "F.Cu") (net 4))
 (segment (start 166.475 30.47237) (end 166.525 30.52237) (width 0.2) (layer "F.Cu") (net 4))
 (segment (start 165.424 36.599) (end 165.424 33.681) (width 0.2) (layer "F.Cu") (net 4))
 (segment (start 174.346 38.801) (end 174.346 41.719) (width 0.2) (layer "F.Cu") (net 4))
 (segment (start 166.475 21.375) (end 166.3 21.2) (width 0.2) (layer "F.Cu") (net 4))
 (segment (start 173.245 32.58) (end 174.346 33.681) (width 0.2) (layer "F.Cu") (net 4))
 (segment (start 174.925 46.26) (end 174.925 44.5) (width 0.2) (layer "F.Cu") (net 4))
 (segment (start 166.475 30.47237) (end 166.475 21.375) (width 0.2) (layer "F.Cu") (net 4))
 (segment (start 173.245 37.7) (end 174.346 38.801) (width 0.2) (layer "F.Cu") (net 4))
 (segment (start 165.424 33.681) (end 166.525 32.58) (width 0.2) (layer "F.Cu") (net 4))
 (segment (start 172.144 43.844) (end 172.144 45.1039) (width 0.2) (layer "F.Cu") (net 4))
 (segment (start 174.346 33.681) (end 174.346 36.599) (width 0.2) (layer "F.Cu") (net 4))
 (segment (start 166.525 42.82) (end 167.626 41.719) (width 0.2) (layer "F.Cu") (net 4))
 (segment (start 166.525 30.52237) (end 166.525 32.58) (width 0.2) (layer "F.Cu") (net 4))
 (segment (start 172.144 45.1039) (end 170.4079 46.84) (width 0.2) (layer "F.Cu") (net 4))
 (segment (start 167.626 41.719) (end 167.626 38.801) (width 0.2) (layer "F.Cu") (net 4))
 (segment (start 173.175 48.01) (end 174.346 46.839) (width 0.2) (layer "F.Cu") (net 4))
 (segment (start 167.626 38.801) (end 166.525 37.7) (width 0.2) (layer "F.Cu") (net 4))
 (segment (start 174.346 46.839) (end 174.346 43.844) (width 0.2) (layer "F.Cu") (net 4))
 (segment (start 174.346 43.844) (end 172.144 43.844) (width 0.2) (layer "F.Cu") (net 4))
 (segment (start 174.925 44.5) (end 173.245 42.82) (width 0.2) (layer "F.Cu") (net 4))
 (segment (start 166.525 42.82) (end 167.625 43.92) (width 0.2) (layer "F.Cu") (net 4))
 (segment (start 167.181 47.284) (end 166.525 47.94) (width 0.2) (layer "F.Cu") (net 4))
 (segment (start 174.346 36.599) (end 173.245 37.7) (width 0.2) (layer "F.Cu") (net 4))
 (segment (start 173.175 48.01) (end 174.925 46.26) (width 0.2) (layer "F.Cu") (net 4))
 (segment (start 170.4079 46.84) (end 167.625 46.84) (width 0.2) (layer "F.Cu") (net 4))
 (segment (start 156.125 21.2) (end 157.20263 21.2) (width 0.2) (layer "F.Cu") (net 4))
 (segment (start 166.525 37.7) (end 165.424 36.599) (width 0.2) (layer "F.Cu") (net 4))
 (segment (start 169.745 32.58) (end 168.275 32.58) (width 0.2) (layer "F.Cu") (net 12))
 (segment (start 168.275 32.58) (end 166.525 34.33) (width 0.2) (layer "F.Cu") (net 12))
 (segment (start 164.126 38.801) (end 163.025 37.7) (width 0.2) (layer "F.Cu") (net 1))
 (segment (start 166.525 44.57) (end 164.126 42.171) (width 0.2) (layer "F.Cu") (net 1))
 (segment (start 164.126 42.171) (end 164.126 38.801) (width 0.2) (layer "F.Cu") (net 1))
 (segment (start 166.525 49.69) (end 165.4 48.565) (width 0.2) (layer "F.Cu") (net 10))
 (segment (start 165.4 45.195) (end 163.025 42.82) (width 0.2) (layer "F.Cu") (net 10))
 (segment (start 165.4 48.565) (end 165.4 45.195) (width 0.2) (layer "F.Cu") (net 10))
 (segment (start 172.449 49.034) (end 173.175 49.76) (width 0.2) (layer "F.Cu") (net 7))
 (segment (start 165.501 50.416) (end 167.626 50.416) (width 0.2) (layer "F.Cu") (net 7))
 (segment (start 167.626 50.416) (end 168.574 49.468) (width 0.2) (layer "F.Cu") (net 7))
 (segment (start 168.574 49.468) (end 168.574 49.034) (width 0.2) (layer "F.Cu") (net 7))
 (segment (start 163.025 47.94) (end 165.501 50.416) (width 0.2) (layer "F.Cu") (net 7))
 (segment (start 168.574 49.034) (end 172.449 49.034) (width 0.2) (layer "F.Cu") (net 7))
 (segment (start 169.675 48.01) (end 169.805 48.01) (width 0.2) (layer "F.Cu") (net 6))
 (segment (start 169.805 48.01) (end 173.245 44.57) (width 0.2) (layer "F.Cu") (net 6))
 (segment (start 173.115 34.33) (end 169.745 37.7) (width 0.2) (layer "F.Cu") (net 8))
 (segment (start 173.245 34.33) (end 173.115 34.33) (width 0.2) (layer "F.Cu") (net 8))
 (segment (start 170.574 45.676) (end 169.024 45.676) (width 0.2) (layer "F.Cu") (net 9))
 (segment (start 168.243 33.707) (end 168.644 33.306) (width 0.2) (layer "F.Cu") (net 9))
 (segment (start 168.243 44.895) (end 168.243 33.707) (width 0.2) (layer "F.Cu") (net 9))
 (segment (start 171.025 19.9) (end 142.185 19.9) (width 0.2) (layer "F.Cu") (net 9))
 (segment (start 142.185 19.9) (end 140.885 21.2) (width 0.2) (layer "F.Cu") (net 9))
 (segment (start 168.644 33.306) (end 170.846 33.306) (width 0.2) (layer "F.Cu") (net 9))
 (segment (start 169.024 45.676) (end 168.243 44.895) (width 0.2) (layer "F.Cu") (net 9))
 (segment (start 171.247 41.448) (end 171.247 45.003) (width 0.2) (layer "F.Cu") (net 9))
 (segment (start 170.846 33.306) (end 171.025 33.127) (width 0.2) (layer "F.Cu") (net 9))
 (segment (start 171.247 45.003) (end 170.574 45.676) (width 0.2) (layer "F.Cu") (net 9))
 (segment (start 171.025 33.127) (end 171.025 19.9) (width 0.2) (layer "F.Cu") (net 9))
 (segment (start 173.245 39.45) (end 171.247 41.448) (width 0.2) (layer "F.Cu") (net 9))
 (segment (start 144.71 47.86) (end 144.71 27.565) (width 0.2) (layer "F.Cu") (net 11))
 (segment (start 144.71 27.565) (end 140.885 23.74) (width 0.2) (layer "F.Cu") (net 11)))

